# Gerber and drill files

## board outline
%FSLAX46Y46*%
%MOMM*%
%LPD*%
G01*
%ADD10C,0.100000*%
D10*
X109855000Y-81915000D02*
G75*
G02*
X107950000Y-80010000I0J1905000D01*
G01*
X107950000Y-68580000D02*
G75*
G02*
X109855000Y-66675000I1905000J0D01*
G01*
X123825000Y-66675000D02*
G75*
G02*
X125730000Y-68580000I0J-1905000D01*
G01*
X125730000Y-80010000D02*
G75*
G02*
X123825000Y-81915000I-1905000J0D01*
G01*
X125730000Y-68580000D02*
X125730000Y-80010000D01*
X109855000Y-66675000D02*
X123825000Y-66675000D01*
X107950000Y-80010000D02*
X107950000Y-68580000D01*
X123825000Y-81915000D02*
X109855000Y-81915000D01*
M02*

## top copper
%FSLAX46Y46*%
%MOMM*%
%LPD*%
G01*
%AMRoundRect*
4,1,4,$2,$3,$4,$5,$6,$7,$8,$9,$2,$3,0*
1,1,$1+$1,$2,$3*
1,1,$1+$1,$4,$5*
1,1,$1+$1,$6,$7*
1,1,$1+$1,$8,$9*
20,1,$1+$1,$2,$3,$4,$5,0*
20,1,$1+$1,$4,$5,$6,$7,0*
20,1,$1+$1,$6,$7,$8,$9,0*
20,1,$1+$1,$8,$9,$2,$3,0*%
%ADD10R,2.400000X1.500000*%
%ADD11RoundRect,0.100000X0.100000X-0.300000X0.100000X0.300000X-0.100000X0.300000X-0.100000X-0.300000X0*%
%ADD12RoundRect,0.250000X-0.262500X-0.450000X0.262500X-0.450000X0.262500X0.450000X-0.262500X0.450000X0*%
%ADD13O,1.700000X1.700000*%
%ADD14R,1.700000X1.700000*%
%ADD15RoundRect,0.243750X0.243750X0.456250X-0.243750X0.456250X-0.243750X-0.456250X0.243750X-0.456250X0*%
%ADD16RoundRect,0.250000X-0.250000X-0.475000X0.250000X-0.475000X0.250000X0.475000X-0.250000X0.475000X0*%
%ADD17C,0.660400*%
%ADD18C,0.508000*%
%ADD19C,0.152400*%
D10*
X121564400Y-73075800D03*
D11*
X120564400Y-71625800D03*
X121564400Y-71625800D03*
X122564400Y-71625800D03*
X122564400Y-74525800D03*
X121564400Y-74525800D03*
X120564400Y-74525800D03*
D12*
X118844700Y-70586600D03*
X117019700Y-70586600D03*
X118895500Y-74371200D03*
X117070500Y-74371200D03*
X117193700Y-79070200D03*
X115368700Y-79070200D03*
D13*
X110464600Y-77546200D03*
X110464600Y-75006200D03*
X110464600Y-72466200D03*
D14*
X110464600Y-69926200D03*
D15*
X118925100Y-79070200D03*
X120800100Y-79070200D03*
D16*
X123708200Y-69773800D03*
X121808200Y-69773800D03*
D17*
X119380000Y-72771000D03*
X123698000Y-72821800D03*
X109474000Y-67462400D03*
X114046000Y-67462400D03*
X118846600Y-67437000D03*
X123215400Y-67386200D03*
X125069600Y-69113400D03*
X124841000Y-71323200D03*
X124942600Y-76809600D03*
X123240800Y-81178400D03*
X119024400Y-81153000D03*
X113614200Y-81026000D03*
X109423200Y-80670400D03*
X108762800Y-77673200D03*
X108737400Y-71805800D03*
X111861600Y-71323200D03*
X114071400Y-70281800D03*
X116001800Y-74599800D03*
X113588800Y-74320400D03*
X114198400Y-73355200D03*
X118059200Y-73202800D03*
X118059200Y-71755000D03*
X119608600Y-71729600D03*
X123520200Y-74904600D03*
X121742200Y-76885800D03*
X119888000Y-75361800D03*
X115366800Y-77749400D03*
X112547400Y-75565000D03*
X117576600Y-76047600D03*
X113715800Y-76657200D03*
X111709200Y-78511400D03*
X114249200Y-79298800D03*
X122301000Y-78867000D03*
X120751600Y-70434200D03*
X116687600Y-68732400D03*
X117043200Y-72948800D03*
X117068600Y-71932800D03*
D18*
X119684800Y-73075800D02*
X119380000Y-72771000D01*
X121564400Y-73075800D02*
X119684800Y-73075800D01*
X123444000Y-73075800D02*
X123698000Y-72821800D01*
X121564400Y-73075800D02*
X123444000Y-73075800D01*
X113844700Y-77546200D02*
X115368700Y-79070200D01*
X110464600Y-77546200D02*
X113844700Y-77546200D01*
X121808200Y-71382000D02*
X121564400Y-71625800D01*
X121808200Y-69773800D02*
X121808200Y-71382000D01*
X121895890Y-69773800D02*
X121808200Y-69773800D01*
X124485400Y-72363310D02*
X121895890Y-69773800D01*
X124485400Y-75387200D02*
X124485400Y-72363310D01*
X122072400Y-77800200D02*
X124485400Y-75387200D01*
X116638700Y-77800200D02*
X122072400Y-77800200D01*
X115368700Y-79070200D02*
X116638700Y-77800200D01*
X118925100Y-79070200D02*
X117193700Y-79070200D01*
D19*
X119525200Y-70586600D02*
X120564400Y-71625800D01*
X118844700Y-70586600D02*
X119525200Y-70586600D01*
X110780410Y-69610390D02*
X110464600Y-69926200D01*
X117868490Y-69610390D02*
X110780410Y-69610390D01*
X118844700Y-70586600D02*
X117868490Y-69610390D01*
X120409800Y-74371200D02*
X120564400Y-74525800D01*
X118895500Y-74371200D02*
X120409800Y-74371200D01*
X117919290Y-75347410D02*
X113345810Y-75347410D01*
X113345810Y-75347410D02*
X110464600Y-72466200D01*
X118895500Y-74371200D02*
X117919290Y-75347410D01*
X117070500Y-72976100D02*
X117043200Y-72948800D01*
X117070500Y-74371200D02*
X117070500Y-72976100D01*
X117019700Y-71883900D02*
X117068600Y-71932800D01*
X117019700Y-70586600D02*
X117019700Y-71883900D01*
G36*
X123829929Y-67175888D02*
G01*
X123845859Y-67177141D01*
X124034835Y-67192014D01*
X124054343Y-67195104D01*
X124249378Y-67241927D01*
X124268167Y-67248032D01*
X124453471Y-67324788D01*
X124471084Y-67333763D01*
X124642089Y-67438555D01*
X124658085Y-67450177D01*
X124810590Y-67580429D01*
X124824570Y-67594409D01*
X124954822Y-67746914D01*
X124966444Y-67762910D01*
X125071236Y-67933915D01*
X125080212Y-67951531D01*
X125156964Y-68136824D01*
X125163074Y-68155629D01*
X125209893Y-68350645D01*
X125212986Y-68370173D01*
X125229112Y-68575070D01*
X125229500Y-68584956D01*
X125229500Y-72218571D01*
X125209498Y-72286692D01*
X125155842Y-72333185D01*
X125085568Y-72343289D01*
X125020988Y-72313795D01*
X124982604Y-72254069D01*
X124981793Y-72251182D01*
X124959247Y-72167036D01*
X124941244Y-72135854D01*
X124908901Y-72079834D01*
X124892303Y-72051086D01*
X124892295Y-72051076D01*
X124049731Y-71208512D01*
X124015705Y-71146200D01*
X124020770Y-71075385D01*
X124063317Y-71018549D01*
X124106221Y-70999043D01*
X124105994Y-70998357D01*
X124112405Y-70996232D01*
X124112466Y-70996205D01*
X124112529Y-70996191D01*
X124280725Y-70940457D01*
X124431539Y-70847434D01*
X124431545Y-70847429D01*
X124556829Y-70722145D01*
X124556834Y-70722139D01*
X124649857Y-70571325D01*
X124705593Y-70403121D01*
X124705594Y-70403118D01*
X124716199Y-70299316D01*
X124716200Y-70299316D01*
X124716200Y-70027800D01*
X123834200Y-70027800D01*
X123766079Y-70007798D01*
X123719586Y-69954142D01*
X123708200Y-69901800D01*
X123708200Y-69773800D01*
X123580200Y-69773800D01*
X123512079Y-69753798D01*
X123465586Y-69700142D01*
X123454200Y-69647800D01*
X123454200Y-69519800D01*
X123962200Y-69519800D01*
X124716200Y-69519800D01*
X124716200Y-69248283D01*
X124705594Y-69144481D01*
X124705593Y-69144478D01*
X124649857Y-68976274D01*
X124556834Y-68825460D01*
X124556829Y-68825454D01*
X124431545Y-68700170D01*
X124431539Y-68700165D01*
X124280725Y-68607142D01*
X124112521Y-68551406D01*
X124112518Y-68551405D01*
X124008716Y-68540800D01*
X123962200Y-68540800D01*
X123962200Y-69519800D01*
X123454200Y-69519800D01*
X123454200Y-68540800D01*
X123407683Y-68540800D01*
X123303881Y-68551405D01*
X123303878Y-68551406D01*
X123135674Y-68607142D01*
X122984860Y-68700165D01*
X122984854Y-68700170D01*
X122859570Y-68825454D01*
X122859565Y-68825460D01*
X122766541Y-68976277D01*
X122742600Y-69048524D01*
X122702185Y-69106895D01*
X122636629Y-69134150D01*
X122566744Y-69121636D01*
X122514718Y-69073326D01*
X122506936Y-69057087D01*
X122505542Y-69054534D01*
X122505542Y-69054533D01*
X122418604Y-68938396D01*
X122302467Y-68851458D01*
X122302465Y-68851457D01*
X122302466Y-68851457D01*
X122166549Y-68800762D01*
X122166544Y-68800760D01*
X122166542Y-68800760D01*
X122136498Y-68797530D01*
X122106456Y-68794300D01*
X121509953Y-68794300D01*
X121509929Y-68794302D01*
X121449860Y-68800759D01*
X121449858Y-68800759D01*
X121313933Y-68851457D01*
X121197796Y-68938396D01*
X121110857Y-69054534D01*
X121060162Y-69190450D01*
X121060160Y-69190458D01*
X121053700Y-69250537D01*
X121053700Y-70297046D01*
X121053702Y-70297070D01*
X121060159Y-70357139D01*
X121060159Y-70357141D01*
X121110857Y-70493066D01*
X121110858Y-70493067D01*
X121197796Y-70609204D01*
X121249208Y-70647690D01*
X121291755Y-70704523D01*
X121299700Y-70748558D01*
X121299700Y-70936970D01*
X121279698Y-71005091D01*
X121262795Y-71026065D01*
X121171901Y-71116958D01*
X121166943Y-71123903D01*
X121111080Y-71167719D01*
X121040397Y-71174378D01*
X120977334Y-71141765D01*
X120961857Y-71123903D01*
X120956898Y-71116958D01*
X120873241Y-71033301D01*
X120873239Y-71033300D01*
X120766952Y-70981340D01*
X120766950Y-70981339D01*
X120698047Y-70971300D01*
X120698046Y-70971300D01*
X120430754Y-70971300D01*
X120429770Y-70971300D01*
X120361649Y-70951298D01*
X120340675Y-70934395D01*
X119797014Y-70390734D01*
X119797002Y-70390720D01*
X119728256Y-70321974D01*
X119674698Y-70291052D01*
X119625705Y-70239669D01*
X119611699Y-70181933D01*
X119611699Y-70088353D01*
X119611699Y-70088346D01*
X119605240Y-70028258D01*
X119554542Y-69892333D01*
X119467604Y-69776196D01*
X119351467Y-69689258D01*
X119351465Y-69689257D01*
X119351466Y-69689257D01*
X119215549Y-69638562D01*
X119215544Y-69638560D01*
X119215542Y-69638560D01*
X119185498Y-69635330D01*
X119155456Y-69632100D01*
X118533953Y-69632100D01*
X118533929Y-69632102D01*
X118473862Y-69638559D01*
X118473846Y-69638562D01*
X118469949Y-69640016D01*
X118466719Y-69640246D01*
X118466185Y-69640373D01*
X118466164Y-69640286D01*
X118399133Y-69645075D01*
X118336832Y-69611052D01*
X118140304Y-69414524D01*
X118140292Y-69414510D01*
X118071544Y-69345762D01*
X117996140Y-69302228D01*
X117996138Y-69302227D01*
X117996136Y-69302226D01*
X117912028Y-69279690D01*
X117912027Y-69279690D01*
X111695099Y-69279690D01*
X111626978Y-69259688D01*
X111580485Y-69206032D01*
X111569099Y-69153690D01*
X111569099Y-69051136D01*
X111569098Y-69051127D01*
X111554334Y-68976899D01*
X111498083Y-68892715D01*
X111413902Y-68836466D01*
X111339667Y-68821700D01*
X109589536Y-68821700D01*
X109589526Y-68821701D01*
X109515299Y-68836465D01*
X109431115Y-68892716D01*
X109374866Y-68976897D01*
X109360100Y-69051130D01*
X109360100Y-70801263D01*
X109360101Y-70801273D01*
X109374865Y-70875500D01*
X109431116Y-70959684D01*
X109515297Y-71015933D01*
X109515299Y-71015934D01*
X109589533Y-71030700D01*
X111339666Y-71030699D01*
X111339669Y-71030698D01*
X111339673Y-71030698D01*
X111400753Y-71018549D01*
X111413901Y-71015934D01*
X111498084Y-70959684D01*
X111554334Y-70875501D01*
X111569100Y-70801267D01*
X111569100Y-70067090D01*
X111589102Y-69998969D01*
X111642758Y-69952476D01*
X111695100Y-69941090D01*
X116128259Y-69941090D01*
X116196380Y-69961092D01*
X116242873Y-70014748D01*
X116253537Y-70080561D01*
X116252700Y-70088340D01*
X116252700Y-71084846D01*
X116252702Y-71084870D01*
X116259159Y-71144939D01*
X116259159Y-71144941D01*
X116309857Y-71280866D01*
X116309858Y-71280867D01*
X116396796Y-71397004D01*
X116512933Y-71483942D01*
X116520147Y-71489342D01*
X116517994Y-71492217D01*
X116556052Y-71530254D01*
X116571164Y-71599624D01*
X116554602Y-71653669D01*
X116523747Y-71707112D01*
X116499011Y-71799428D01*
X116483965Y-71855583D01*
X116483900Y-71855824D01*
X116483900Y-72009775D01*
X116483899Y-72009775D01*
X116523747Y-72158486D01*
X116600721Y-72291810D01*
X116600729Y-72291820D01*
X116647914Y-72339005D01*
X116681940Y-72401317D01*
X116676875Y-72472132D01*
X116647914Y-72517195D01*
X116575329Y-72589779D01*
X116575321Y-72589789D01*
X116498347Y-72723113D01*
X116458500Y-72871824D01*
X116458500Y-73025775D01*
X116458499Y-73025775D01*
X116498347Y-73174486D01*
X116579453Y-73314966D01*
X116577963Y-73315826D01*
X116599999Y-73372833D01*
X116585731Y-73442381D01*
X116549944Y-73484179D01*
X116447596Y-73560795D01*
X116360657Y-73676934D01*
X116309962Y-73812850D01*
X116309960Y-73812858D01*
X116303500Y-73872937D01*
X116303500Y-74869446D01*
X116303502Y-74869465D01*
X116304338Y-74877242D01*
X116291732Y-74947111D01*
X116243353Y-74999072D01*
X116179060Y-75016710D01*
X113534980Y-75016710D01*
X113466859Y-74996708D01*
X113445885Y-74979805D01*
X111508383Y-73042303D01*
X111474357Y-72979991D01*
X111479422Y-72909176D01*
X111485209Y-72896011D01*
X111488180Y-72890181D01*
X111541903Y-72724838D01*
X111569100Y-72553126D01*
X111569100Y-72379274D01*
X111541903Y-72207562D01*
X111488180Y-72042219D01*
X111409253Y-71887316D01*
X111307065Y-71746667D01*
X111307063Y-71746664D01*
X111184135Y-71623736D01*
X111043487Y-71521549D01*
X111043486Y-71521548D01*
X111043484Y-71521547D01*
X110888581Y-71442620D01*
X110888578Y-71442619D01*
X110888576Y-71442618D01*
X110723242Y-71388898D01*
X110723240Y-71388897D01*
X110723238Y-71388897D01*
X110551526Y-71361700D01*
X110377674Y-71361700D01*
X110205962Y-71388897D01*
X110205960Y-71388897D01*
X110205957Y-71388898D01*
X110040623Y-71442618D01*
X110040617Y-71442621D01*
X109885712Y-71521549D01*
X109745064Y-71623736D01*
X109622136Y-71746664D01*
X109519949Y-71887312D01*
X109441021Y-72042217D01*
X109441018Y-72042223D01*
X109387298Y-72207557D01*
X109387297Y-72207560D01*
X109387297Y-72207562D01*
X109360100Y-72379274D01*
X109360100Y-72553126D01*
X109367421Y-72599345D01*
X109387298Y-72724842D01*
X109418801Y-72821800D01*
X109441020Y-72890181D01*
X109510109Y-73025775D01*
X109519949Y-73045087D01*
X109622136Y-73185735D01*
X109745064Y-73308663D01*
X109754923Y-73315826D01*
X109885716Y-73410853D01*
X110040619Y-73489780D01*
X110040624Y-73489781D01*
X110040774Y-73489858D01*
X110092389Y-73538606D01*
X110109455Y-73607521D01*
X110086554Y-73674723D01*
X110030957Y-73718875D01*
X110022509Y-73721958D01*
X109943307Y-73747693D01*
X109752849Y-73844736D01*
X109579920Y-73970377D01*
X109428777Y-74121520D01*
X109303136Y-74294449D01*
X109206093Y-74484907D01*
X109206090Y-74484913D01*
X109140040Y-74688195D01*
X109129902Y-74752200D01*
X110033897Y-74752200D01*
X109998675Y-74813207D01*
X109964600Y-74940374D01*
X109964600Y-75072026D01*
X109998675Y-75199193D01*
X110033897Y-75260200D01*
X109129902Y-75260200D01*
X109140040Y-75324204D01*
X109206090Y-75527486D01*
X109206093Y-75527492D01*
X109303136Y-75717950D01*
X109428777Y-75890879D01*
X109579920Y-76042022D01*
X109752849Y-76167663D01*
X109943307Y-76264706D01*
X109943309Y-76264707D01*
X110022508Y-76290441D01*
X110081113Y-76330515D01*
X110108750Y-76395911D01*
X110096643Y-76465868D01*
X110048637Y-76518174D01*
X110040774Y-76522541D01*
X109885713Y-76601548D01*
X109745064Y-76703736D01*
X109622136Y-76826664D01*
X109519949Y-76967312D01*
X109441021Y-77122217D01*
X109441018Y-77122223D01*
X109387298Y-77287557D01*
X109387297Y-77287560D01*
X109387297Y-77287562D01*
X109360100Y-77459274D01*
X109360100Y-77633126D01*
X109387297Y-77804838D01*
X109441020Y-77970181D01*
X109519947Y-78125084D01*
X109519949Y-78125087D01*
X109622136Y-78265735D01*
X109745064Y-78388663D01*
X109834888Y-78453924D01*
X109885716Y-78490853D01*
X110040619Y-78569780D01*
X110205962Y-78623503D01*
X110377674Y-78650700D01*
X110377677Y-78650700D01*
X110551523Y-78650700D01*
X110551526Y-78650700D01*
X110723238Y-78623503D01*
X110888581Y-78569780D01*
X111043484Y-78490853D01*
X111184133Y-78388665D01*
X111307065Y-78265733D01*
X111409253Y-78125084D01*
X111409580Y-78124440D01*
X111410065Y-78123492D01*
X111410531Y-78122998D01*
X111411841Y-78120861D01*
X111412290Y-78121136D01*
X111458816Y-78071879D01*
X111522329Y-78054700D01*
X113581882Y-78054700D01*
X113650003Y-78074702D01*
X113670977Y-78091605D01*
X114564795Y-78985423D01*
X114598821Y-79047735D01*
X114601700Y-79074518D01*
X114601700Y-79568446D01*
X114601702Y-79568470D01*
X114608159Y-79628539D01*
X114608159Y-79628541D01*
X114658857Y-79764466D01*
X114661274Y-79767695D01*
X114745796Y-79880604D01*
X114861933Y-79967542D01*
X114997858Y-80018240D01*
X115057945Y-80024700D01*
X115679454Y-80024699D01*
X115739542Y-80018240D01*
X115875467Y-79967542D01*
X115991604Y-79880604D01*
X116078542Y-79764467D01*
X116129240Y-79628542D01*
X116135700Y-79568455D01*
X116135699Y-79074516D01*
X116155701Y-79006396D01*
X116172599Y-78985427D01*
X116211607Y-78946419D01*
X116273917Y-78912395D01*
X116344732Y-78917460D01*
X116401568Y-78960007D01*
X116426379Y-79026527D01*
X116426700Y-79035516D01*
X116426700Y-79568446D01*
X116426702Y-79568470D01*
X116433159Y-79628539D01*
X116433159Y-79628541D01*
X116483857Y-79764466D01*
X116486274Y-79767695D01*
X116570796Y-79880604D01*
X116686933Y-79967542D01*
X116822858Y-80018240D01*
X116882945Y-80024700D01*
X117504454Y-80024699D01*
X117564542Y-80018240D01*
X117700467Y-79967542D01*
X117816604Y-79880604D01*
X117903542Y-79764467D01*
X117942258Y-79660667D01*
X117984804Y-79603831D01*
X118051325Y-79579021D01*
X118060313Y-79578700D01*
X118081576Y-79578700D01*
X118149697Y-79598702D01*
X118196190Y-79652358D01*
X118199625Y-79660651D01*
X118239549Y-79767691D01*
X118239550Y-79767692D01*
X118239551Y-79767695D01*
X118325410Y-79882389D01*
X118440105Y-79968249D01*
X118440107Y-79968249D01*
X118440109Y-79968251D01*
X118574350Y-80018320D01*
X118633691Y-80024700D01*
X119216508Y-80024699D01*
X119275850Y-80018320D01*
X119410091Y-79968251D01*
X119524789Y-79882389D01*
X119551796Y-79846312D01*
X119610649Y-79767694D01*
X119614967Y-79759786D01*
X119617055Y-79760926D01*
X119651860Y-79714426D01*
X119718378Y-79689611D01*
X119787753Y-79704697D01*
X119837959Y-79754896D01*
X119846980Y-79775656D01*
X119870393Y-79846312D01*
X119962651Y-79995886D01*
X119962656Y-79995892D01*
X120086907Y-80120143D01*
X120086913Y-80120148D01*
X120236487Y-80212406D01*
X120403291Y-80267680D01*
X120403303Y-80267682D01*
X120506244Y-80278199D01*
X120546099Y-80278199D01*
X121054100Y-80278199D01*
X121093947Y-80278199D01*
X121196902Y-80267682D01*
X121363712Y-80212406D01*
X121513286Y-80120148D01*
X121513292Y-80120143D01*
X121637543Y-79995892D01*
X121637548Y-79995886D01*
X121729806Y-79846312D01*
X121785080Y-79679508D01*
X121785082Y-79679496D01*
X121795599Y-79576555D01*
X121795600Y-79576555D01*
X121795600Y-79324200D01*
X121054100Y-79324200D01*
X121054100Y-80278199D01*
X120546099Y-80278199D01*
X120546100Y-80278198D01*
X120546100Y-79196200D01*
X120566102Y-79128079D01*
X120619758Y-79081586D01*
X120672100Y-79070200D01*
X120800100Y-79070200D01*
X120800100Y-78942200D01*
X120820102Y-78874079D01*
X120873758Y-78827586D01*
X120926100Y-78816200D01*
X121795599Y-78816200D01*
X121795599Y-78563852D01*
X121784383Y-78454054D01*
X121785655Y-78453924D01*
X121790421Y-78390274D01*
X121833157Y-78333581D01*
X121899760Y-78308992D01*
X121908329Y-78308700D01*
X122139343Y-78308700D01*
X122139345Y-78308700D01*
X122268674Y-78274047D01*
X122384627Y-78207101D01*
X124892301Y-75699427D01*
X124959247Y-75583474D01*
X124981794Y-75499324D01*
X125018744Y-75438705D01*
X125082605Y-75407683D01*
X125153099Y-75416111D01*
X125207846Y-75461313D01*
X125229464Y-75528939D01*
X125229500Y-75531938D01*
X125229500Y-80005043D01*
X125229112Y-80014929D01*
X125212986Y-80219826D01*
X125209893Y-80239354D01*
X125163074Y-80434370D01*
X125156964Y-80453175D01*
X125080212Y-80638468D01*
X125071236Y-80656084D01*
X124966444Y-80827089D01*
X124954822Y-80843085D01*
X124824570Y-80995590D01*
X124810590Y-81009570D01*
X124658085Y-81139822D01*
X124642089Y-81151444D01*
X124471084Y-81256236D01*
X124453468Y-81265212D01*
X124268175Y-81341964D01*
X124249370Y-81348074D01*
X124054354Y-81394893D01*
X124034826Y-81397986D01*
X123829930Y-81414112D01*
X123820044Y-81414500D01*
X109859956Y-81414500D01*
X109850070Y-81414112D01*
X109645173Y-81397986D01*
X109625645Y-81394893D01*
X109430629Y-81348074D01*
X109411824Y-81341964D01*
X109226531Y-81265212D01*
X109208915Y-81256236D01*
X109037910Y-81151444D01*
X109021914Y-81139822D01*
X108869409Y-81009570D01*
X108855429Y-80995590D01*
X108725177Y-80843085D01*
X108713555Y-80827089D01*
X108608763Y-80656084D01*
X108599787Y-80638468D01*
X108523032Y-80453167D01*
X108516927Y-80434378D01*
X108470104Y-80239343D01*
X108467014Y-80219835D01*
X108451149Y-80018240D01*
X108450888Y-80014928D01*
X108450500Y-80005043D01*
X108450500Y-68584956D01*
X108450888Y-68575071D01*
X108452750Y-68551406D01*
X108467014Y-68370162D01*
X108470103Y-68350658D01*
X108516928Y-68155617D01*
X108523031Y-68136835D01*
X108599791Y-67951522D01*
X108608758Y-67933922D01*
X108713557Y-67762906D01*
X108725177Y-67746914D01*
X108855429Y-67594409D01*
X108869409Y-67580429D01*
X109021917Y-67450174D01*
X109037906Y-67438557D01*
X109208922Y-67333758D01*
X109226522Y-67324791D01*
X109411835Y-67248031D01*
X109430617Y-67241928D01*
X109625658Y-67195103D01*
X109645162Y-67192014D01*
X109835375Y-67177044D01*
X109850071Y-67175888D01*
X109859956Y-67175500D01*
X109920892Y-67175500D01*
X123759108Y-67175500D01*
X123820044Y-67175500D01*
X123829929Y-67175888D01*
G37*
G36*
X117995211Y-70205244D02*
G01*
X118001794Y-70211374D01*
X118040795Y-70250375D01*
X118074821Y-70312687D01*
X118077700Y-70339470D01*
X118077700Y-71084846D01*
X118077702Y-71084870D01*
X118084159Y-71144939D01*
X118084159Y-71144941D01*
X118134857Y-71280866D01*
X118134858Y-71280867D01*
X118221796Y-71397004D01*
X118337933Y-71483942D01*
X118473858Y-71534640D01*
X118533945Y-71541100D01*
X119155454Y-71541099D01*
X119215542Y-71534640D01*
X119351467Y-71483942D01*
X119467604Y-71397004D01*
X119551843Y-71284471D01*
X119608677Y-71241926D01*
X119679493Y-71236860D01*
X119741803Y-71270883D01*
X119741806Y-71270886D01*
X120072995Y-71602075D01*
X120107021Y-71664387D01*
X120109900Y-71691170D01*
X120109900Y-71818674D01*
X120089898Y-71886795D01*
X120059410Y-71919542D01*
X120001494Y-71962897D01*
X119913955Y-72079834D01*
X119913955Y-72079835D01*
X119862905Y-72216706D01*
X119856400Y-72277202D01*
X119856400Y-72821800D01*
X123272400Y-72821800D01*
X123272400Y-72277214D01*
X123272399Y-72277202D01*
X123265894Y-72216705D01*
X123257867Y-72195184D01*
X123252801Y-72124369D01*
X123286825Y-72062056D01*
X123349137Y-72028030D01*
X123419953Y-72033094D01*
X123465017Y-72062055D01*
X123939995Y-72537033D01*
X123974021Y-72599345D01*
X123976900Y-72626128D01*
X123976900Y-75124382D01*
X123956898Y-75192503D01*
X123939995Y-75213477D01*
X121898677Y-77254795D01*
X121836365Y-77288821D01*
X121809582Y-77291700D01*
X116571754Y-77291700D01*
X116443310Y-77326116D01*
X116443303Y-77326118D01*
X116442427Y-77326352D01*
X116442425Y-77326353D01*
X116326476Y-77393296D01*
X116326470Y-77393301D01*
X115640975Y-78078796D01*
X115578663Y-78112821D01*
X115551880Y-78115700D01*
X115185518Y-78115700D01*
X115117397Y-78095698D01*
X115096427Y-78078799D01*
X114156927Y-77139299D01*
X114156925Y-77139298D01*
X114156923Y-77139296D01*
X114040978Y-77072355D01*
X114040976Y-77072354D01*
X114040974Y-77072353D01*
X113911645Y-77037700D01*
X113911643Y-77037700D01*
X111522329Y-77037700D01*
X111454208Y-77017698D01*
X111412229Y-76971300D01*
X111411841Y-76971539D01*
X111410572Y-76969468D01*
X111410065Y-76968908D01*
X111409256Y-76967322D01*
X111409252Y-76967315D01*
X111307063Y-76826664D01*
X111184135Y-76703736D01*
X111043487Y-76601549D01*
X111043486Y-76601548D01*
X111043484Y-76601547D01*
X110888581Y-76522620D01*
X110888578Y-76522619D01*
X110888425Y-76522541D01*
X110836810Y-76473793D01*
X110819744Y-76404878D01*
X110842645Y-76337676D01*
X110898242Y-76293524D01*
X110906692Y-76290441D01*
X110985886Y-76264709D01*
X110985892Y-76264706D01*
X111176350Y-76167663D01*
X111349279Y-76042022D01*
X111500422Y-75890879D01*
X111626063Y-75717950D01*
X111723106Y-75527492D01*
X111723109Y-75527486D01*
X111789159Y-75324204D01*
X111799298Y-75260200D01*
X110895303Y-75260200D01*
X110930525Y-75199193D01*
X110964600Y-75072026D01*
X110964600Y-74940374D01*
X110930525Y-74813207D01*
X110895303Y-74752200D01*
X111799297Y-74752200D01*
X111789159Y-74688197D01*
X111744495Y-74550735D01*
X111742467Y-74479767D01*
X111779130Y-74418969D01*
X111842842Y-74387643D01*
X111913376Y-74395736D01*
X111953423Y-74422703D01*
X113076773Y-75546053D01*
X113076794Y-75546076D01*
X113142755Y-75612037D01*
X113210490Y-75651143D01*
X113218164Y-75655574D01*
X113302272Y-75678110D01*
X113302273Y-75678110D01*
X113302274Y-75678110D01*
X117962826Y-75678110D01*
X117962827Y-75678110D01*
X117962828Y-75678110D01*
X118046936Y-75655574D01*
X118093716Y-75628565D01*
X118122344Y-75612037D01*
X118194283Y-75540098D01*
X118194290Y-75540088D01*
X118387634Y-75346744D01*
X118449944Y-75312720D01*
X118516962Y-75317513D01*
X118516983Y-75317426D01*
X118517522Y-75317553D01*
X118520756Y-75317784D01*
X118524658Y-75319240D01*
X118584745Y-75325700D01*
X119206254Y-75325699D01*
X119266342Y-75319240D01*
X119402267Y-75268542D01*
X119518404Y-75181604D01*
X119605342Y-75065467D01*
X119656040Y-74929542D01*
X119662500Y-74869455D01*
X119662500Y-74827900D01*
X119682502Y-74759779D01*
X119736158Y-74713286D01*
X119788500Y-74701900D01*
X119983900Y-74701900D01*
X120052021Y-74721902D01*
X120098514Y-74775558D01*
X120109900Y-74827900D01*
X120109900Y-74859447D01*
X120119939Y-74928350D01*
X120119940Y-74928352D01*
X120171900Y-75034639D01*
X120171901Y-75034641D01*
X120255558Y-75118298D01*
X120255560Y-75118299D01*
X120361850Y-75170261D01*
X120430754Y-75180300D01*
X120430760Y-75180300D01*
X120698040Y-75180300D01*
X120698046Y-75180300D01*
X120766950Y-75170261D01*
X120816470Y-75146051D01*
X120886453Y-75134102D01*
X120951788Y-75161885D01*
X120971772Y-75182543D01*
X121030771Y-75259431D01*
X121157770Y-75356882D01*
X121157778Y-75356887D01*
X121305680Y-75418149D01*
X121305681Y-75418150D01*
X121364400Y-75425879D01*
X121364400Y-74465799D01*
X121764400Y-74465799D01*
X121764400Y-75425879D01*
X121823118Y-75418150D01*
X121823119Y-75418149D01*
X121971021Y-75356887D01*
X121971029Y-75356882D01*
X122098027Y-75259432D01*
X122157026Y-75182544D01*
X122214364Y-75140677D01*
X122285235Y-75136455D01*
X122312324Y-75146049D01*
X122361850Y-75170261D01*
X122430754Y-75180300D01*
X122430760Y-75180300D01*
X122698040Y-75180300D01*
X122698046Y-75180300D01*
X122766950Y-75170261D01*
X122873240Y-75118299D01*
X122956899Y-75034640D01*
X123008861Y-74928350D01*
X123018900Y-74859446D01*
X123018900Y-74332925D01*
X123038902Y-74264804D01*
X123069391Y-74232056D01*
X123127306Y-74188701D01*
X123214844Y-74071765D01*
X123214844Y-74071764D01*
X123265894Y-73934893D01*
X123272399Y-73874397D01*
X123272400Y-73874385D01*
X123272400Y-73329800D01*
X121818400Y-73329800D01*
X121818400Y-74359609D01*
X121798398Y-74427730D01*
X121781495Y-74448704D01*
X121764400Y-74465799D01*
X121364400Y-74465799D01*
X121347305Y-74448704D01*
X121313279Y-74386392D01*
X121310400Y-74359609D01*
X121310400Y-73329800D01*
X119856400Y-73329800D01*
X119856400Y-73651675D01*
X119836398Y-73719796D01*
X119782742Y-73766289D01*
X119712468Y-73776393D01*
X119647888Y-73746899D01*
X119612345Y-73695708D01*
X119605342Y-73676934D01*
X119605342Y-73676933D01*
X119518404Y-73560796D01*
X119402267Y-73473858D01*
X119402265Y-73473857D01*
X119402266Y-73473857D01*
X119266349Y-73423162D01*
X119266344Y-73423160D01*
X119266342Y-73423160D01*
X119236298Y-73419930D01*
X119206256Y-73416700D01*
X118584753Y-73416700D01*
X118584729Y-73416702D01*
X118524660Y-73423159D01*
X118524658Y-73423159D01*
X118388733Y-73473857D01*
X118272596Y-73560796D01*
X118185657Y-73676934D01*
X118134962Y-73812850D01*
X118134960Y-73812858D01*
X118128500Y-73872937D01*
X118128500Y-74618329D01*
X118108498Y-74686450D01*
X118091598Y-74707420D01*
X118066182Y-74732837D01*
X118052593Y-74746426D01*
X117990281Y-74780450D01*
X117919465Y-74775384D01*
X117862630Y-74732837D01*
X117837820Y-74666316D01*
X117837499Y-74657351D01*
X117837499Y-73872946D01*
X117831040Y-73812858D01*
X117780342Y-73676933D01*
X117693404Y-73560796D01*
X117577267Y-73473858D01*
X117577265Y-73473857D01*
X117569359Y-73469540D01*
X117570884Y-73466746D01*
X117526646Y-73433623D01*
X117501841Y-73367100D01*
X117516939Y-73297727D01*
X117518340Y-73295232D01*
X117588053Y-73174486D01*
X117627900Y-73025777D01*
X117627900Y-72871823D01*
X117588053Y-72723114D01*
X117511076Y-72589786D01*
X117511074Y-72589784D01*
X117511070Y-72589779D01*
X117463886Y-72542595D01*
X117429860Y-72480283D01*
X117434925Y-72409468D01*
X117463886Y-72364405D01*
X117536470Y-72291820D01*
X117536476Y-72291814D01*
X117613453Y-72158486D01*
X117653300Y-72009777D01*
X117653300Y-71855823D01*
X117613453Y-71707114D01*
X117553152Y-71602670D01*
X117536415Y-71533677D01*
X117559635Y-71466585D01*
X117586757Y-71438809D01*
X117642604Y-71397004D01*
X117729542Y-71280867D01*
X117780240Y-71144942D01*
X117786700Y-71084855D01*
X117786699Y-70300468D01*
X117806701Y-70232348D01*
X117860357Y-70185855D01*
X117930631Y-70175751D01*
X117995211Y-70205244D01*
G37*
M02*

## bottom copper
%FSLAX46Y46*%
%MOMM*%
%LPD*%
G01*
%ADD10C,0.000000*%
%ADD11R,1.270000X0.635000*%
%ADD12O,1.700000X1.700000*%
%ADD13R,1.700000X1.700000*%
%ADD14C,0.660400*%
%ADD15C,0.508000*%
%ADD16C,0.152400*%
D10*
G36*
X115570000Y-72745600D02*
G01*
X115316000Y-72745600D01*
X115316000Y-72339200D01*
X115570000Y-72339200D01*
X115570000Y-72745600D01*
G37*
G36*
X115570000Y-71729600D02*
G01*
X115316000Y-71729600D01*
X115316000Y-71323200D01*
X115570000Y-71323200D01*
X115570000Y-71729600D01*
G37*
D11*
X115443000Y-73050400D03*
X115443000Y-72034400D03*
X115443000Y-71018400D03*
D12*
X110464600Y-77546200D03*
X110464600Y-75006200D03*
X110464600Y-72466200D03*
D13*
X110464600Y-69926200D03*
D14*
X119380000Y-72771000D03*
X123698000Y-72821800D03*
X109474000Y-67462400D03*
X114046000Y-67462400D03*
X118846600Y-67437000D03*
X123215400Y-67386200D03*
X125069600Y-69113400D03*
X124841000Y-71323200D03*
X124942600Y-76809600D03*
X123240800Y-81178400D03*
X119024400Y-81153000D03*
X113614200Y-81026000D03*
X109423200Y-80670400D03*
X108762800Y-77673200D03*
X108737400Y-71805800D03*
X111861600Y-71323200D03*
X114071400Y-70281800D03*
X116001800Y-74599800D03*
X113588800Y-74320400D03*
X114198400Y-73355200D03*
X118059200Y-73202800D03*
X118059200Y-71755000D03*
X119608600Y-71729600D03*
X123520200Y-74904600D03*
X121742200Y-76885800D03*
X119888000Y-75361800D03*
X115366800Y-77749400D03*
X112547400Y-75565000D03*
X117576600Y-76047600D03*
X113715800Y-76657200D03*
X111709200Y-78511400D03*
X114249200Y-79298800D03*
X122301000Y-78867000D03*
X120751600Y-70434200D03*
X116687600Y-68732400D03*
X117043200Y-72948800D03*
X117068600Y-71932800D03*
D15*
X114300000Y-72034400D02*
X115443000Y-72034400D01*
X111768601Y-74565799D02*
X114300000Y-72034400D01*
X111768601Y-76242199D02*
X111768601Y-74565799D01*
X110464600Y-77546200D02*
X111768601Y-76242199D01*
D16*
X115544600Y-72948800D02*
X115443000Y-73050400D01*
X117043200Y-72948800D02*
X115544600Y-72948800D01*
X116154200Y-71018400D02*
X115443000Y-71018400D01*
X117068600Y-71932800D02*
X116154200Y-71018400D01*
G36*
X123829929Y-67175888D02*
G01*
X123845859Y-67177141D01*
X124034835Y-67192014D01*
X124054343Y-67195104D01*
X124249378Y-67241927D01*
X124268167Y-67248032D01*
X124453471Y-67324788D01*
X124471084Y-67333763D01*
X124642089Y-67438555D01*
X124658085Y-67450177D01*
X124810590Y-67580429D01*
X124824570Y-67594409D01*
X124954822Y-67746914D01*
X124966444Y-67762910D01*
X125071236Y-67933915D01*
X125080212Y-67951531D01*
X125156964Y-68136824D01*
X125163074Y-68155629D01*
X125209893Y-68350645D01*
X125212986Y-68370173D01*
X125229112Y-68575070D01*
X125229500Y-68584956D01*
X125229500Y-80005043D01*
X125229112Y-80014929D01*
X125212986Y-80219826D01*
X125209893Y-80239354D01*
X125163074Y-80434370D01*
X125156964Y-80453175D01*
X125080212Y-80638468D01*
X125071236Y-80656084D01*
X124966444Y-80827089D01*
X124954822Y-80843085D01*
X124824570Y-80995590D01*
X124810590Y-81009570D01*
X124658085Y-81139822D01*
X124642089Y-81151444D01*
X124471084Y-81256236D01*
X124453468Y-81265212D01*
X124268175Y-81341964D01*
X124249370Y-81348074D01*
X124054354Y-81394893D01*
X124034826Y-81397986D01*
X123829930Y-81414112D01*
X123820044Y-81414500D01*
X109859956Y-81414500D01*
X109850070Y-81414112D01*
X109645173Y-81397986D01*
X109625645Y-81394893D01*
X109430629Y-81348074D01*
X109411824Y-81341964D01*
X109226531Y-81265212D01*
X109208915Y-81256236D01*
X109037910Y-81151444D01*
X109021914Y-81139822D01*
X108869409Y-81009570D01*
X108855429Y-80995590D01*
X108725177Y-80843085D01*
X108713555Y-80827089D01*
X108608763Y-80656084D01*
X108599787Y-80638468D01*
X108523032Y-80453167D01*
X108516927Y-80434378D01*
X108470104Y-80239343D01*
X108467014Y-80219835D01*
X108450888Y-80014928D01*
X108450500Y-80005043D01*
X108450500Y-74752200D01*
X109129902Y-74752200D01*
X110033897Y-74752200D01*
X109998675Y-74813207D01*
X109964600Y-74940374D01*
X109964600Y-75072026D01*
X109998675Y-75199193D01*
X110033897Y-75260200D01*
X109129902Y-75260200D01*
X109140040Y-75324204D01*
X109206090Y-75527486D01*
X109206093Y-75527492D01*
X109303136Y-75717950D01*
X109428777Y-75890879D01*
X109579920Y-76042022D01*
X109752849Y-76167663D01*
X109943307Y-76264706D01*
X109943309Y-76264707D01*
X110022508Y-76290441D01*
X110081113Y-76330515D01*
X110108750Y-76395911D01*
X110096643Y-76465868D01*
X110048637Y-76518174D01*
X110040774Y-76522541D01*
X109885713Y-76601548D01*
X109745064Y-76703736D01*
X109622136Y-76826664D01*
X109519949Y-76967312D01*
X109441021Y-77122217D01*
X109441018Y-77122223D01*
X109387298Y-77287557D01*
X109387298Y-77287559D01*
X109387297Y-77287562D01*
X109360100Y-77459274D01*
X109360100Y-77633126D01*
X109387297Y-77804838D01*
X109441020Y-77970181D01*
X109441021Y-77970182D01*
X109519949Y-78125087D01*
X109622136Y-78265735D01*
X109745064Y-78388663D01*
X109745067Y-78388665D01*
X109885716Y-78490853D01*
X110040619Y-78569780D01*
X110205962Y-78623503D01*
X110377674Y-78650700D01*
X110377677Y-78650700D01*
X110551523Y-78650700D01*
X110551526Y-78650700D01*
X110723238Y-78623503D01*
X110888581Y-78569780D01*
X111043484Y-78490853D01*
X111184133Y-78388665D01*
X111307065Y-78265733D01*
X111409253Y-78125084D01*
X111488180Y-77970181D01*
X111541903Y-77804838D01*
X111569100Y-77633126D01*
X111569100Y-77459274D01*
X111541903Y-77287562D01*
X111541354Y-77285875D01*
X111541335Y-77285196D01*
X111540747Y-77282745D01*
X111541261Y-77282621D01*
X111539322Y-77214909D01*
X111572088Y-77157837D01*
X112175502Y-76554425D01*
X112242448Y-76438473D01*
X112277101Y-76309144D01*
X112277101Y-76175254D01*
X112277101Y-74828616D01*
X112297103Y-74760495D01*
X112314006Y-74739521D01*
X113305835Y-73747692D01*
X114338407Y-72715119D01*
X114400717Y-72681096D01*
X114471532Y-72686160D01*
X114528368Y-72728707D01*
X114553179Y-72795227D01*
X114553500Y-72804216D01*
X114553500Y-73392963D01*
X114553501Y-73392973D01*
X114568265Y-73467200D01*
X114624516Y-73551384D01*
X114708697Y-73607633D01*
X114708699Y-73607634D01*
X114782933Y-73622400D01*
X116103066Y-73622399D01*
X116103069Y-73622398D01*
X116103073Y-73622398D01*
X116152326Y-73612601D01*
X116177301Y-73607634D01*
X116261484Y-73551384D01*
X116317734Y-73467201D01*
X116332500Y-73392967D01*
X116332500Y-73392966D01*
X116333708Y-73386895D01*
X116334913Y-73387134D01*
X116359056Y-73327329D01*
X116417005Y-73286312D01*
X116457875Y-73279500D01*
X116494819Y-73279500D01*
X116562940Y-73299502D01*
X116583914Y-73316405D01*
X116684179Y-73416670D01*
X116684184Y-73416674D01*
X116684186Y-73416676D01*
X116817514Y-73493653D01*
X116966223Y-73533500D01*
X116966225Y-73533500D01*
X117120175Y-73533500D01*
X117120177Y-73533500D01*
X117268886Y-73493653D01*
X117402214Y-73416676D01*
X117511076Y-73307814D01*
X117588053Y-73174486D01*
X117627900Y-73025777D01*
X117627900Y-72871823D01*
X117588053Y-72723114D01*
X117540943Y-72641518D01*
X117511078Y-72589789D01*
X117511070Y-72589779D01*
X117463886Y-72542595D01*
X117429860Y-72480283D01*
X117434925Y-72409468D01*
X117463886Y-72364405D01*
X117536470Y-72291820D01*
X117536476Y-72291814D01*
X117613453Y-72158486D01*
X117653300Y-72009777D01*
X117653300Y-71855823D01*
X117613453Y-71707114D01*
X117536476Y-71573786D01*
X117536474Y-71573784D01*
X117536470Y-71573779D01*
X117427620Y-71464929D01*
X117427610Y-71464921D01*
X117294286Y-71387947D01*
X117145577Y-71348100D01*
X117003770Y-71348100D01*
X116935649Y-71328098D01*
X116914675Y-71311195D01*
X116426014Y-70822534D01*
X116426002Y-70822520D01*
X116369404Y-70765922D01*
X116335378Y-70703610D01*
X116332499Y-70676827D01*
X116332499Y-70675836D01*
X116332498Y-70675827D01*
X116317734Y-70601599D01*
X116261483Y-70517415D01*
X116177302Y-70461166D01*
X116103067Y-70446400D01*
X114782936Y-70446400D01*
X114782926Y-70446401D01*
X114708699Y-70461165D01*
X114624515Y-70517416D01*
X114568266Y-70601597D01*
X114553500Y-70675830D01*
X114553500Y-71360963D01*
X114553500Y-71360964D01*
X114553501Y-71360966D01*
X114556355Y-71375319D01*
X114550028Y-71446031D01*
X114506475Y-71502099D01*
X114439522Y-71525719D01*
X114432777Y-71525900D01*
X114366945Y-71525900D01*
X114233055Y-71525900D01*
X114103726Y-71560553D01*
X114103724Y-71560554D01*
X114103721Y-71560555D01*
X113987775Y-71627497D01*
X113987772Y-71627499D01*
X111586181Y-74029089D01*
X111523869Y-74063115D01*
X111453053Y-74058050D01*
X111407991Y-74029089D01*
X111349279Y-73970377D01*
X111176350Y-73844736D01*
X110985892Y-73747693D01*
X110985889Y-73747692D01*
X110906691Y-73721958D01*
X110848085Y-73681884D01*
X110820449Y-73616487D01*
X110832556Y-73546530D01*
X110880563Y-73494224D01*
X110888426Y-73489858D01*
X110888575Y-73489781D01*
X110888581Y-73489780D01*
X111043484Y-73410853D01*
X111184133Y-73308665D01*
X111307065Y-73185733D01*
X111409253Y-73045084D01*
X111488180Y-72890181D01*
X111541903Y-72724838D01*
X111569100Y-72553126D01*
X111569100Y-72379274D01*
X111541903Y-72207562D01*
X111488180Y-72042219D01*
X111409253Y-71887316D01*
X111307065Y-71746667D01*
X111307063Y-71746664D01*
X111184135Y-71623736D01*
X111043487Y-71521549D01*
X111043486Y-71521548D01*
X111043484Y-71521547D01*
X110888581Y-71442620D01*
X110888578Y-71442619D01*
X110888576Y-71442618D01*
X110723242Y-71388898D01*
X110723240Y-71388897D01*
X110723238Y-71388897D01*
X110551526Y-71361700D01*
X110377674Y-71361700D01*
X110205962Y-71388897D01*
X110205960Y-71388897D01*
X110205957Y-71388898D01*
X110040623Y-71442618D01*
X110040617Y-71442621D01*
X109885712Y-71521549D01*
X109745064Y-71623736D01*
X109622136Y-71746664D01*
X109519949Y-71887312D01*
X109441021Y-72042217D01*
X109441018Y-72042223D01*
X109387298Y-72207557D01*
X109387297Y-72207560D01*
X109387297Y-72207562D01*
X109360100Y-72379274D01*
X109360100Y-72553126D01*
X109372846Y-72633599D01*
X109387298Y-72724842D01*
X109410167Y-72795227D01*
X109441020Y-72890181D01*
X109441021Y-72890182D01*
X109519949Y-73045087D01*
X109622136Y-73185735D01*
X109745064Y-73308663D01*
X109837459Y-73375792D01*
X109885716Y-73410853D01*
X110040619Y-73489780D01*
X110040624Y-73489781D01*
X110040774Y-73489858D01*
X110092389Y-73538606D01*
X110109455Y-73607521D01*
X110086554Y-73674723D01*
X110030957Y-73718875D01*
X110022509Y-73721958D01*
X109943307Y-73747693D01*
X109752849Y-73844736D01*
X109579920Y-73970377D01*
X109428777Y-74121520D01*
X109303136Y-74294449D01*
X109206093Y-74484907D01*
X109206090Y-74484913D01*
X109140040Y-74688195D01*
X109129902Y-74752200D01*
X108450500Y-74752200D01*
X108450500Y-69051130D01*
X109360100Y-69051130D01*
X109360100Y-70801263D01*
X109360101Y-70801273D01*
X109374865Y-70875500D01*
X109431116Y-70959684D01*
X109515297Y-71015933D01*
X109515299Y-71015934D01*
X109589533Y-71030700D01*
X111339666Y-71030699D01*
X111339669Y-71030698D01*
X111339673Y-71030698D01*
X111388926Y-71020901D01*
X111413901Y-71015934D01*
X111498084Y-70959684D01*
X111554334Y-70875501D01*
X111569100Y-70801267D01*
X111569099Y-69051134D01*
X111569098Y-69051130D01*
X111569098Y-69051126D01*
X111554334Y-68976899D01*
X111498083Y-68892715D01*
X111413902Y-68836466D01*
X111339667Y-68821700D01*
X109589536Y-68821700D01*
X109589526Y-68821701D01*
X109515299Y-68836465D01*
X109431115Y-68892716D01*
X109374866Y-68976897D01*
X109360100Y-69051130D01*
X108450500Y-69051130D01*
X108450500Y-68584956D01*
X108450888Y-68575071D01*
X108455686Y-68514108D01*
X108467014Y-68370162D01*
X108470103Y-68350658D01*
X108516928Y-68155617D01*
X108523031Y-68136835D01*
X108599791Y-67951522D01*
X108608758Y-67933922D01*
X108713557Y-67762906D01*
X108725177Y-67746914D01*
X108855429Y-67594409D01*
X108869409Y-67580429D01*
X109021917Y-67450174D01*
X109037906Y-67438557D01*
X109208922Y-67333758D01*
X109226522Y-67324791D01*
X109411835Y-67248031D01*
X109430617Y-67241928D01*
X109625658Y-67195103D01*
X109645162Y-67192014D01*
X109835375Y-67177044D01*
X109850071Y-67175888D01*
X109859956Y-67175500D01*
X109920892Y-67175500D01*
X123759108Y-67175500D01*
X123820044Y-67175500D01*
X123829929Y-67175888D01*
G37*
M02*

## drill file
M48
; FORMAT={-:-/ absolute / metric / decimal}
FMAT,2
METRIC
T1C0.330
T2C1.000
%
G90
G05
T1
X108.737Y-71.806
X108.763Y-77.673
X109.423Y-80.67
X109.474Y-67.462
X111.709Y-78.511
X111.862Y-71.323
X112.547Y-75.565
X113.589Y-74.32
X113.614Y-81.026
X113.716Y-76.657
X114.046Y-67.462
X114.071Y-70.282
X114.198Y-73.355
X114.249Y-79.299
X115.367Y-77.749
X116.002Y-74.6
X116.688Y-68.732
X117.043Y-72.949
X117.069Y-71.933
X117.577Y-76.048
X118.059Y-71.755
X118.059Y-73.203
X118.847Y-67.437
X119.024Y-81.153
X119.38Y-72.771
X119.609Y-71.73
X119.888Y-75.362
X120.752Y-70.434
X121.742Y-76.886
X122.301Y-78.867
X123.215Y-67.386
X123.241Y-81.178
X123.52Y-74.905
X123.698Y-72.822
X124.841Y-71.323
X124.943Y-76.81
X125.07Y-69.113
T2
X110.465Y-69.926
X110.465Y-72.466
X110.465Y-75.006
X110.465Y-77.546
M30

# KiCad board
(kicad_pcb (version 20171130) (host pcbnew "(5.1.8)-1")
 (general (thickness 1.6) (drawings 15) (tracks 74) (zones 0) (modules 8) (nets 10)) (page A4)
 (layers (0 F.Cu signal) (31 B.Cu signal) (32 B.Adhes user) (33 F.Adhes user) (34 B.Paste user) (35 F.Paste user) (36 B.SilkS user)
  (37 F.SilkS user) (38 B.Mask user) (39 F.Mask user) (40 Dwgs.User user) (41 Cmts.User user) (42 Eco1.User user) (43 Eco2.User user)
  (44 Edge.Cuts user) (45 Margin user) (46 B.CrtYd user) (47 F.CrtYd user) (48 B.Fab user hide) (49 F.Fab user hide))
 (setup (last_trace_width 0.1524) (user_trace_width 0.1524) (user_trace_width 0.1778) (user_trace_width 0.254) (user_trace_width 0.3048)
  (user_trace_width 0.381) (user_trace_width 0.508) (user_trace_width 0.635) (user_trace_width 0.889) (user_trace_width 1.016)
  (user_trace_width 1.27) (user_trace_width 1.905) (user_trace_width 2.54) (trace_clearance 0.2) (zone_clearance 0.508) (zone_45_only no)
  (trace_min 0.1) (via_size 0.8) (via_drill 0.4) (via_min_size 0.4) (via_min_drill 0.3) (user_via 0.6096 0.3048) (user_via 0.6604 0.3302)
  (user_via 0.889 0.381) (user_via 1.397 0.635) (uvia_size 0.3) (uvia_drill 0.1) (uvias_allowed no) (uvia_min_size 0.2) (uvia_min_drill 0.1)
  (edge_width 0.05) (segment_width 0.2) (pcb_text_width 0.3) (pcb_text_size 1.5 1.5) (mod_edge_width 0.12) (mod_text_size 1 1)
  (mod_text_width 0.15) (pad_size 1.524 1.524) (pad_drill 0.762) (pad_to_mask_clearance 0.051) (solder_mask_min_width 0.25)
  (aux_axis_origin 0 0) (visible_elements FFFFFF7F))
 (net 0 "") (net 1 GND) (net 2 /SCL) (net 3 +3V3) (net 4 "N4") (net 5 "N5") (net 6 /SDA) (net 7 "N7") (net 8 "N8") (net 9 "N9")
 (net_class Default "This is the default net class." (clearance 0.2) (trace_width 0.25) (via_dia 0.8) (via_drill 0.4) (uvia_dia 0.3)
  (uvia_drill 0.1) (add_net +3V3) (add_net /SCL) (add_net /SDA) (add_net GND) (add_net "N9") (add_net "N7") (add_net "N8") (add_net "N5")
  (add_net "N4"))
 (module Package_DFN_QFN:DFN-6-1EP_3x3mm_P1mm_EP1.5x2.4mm (layer F.Cu) (at 121.5644 73.0758 90)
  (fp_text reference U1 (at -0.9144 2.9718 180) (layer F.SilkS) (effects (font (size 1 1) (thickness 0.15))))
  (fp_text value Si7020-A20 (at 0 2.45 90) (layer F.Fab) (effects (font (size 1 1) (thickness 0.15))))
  (pad "" smd roundrect (at 0.375 0.6 90) (size 0.6 0.97) (layers F.Paste) (roundrect_rratio 0.25))
  (pad "" smd roundrect (at 0.375 -0.6 90) (size 0.6 0.97) (layers F.Paste) (roundrect_rratio 0.25))
  (pad "" smd roundrect (at -0.375 0.6 90) (size 0.6 0.97) (layers F.Paste) (roundrect_rratio 0.25))
  (pad "" smd roundrect (at -0.375 -0.6 90) (size 0.6 0.97) (layers F.Paste) (roundrect_rratio 0.25))
  (pad 7 smd rect (at 0 0 90) (size 1.5 2.4) (layers F.Cu F.Mask) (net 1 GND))
  (pad 6 smd roundrect (at 1.45 -1 90) (size 0.8 0.4) (layers F.Cu F.Paste F.Mask) (roundrect_rratio 0.25) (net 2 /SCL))
  (pad 5 smd roundrect (at 1.45 0 90) (size 0.8 0.4) (layers F.Cu F.Paste F.Mask) (roundrect_rratio 0.25) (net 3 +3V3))
  (pad 4 smd roundrect (at 1.45 1 90) (size 0.8 0.4) (layers F.Cu F.Paste F.Mask) (roundrect_rratio 0.25) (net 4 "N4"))
  (pad 3 smd roundrect (at -1.45 1 90) (size 0.8 0.4) (layers F.Cu F.Paste F.Mask) (roundrect_rratio 0.25) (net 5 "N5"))
  (pad 2 smd roundrect (at -1.45 0 90) (size 0.8 0.4) (layers F.Cu F.Paste F.Mask) (roundrect_rratio 0.25) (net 1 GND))
  (pad 1 smd roundrect (at -1.45 -1 90) (size 0.8 0.4) (layers F.Cu F.Paste F.Mask) (roundrect_rratio 0.25) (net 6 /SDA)))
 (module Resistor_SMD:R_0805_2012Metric (layer F.Cu) (at 117.9322 70.5866)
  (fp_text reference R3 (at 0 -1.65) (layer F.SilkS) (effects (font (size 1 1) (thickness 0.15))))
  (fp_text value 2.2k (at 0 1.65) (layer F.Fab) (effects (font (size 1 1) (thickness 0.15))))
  (pad 2 smd roundrect (at 0.9125 0) (size 1.025 1.4) (layers F.Cu F.Paste F.Mask) (roundrect_rratio 0.243902) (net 2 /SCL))
  (pad 1 smd roundrect (at -0.9125 0) (size 1.025 1.4) (layers F.Cu F.Paste F.Mask) (roundrect_rratio 0.243902) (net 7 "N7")))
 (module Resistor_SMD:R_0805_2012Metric (layer F.Cu) (at 117.983 74.3712)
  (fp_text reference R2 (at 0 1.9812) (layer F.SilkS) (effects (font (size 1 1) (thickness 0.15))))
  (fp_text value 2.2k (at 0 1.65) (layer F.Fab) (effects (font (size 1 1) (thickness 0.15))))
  (pad 2 smd roundrect (at 0.9125 0) (size 1.025 1.4) (layers F.Cu F.Paste F.Mask) (roundrect_rratio 0.243902) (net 6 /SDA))
  (pad 1 smd roundrect (at -0.9125 0) (size 1.025 1.4) (layers F.Cu F.Paste F.Mask) (roundrect_rratio 0.243902) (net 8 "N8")))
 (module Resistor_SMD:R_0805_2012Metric (layer F.Cu) (at 116.2812 79.0702)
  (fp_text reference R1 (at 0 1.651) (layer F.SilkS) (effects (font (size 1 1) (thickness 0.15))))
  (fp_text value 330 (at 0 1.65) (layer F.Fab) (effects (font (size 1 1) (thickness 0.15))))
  (pad 2 smd roundrect (at 0.9125 0) (size 1.025 1.4) (layers F.Cu F.Paste F.Mask) (roundrect_rratio 0.243902) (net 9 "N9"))
  (pad 1 smd roundrect (at -0.9125 0) (size 1.025 1.4) (layers F.Cu F.Paste F.Mask) (roundrect_rratio 0.243902) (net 3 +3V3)))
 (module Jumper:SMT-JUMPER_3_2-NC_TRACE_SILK (layer B.Cu) (at 115.443 72.0344 270)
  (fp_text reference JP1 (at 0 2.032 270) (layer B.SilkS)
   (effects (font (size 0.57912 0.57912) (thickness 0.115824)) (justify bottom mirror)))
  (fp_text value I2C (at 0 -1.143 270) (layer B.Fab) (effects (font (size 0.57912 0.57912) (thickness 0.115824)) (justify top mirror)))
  (fp_poly (pts (xy 0.3048 -0.127) (xy 0.7112 -0.127) (xy 0.7112 0.127) (xy 0.3048 0.127)) (layer B.Cu) (width 0))
  (fp_poly (pts (xy -0.7112 -0.127) (xy -0.3048 -0.127) (xy -0.3048 0.127) (xy -0.7112 0.127)) (layer B.Cu) (width 0))
  (pad 3 smd rect (at 1.016 0 270) (size 0.635 1.27) (layers B.Cu B.Mask) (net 8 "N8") (solder_mask_margin 0.1016))
  (pad 2 smd rect (at 0 0 270) (size 0.635 1.27) (layers B.Cu B.Mask) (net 3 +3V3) (solder_mask_margin 0.1016))
  (pad 1 smd rect (at -1.016 0 270) (size 0.635 1.27) (layers B.Cu B.Mask) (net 7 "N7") (solder_mask_margin 0.1016)))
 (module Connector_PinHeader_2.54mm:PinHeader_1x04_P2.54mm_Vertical (layer F.Cu) (at 110.4646 69.9262)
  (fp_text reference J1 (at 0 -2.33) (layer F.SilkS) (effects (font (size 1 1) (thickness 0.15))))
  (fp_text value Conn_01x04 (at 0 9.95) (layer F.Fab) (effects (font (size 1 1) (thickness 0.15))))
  (pad 4 thru_hole oval (at 0 7.62) (size 1.7 1.7) (drill 1) (layers *.Cu *.Mask) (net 3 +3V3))
  (pad 3 thru_hole oval (at 0 5.08) (size 1.7 1.7) (drill 1) (layers *.Cu *.Mask) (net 1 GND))
  (pad 2 thru_hole oval (at 0 2.54) (size 1.7 1.7) (drill 1) (layers *.Cu *.Mask) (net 6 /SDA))
  (pad 1 thru_hole rect (at 0 0) (size 1.7 1.7) (drill 1) (layers *.Cu *.Mask) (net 2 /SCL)))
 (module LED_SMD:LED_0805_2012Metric (layer F.Cu) (at 119.8626 79.0702 180)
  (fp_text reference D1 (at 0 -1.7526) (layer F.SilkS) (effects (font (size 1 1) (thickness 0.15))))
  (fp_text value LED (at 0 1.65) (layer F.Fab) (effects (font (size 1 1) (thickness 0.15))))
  (pad 2 smd roundrect (at 0.9375 0 180) (size 0.975 1.4) (layers F.Cu F.Paste F.Mask) (roundrect_rratio 0.25) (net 9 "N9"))
  (pad 1 smd roundrect (at -0.9375 0 180) (size 0.975 1.4) (layers F.Cu F.Paste F.Mask) (roundrect_rratio 0.25) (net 1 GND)))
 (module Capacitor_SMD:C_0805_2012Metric (layer F.Cu) (at 122.7582 69.7738)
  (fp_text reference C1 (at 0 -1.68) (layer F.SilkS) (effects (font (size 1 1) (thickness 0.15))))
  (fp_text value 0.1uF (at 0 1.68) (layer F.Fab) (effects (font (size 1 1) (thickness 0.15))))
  (pad 2 smd roundrect (at 0.95 0) (size 1 1.45) (layers F.Cu F.Paste F.Mask) (roundrect_rratio 0.25) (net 1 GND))
  (pad 1 smd roundrect (at -0.95 0) (size 1 1.45) (layers F.Cu F.Paste F.Mask) (roundrect_rratio 0.25) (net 3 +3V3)))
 (gr_arc (start 109.855 80.01) (end 107.95 80.01) (angle -90) (layer Edge.Cuts) (width 0.1))
 (gr_arc (start 109.855 68.58) (end 109.855 66.675) (angle -90) (layer Edge.Cuts) (width 0.1))
 (gr_arc (start 123.825 68.58) (end 125.73 68.58) (angle -90) (layer Edge.Cuts) (width 0.1))
 (gr_arc (start 123.825 80.01) (end 123.825 81.915) (angle -90) (layer Edge.Cuts) (width 0.1))
 (gr_line (start 125.73 68.58) (end 125.73 80.01) (layer Edge.Cuts) (width 0.1))
 (gr_line (start 109.855 66.675) (end 123.825 66.675) (layer Edge.Cuts) (width 0.1))
 (gr_line (start 107.95 80.01) (end 107.95 68.58) (layer Edge.Cuts) (width 0.1))
 (gr_line (start 123.825 81.915) (end 109.855 81.915) (layer Edge.Cuts) (width 0.1))
 (via (at 119.38 72.771) (size 0.6604) (drill 0.3302) (layers F.Cu B.Cu) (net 1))
 (via (at 123.698 72.8218) (size 0.6604) (drill 0.3302) (layers F.Cu B.Cu) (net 1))
 (segment (start 119.6848 73.0758) (end 119.38 72.771) (width 0.508) (layer F.Cu) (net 1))
 (segment (start 121.5644 73.0758) (end 119.6848 73.0758) (width 0.508) (layer F.Cu) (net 1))
 (segment (start 123.444 73.0758) (end 123.698 72.8218) (width 0.508) (layer F.Cu) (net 1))
 (segment (start 121.5644 73.0758) (end 123.444 73.0758) (width 0.508) (layer F.Cu) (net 1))
 (via (at 109.474 67.4624) (size 0.6604) (drill 0.3302) (layers F.Cu B.Cu) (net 1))
 (via (at 114.046 67.4624) (size 0.6604) (drill 0.3302) (layers F.Cu B.Cu) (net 1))
 (via (at 118.8466 67.437) (size 0.6604) (drill 0.3302) (layers F.Cu B.Cu) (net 1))
 (via (at 123.2154 67.3862) (size 0.6604) (drill 0.3302) (layers F.Cu B.Cu) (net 1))
 (via (at 125.0696 69.1134) (size 0.6604) (drill 0.3302) (layers F.Cu B.Cu) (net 1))
 (via (at 124.841 71.3232) (size 0.6604) (drill 0.3302) (layers F.Cu B.Cu) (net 1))
 (via (at 124.9426 76.8096) (size 0.6604) (drill 0.3302) (layers F.Cu B.Cu) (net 1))
 (via (at 123.2408 81.1784) (size 0.6604) (drill 0.3302) (layers F.Cu B.Cu) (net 1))
 (via (at 119.0244 81.153) (size 0.6604) (drill 0.3302) (layers F.Cu B.Cu) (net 1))
 (via (at 113.6142 81.026) (size 0.6604) (drill 0.3302) (layers F.Cu B.Cu) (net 1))
 (via (at 109.4232 80.6704) (size 0.6604) (drill 0.3302) (layers F.Cu B.Cu) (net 1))
 (via (at 108.7628 77.6732) (size 0.6604) (drill 0.3302) (layers F.Cu B.Cu) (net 1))
 (via (at 108.7374 71.8058) (size 0.6604) (drill 0.3302) (layers F.Cu B.Cu) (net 1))
 (via (at 111.8616 71.3232) (size 0.6604) (drill 0.3302) (layers F.Cu B.Cu) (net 1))
 (via (at 114.0714 70.2818) (size 0.6604) (drill 0.3302) (layers F.Cu B.Cu) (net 1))
 (via (at 116.0018 74.5998) (size 0.6604) (drill 0.3302) (layers F.Cu B.Cu) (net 1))
 (via (at 113.5888 74.3204) (size 0.6604) (drill 0.3302) (layers F.Cu B.Cu) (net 1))
 (via (at 114.1984 73.3552) (size 0.6604) (drill 0.3302) (layers F.Cu B.Cu) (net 1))
 (via (at 118.0592 73.2028) (size 0.6604) (drill 0.3302) (layers F.Cu B.Cu) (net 1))
 (via (at 118.0592 71.755) (size 0.6604) (drill 0.3302) (layers F.Cu B.Cu) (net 1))
 (via (at 119.6086 71.7296) (size 0.6604) (drill 0.3302) (layers F.Cu B.Cu) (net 1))
 (via (at 123.5202 74.9046) (size 0.6604) (drill 0.3302) (layers F.Cu B.Cu) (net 1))
 (via (at 121.7422 76.8858) (size 0.6604) (drill 0.3302) (layers F.Cu B.Cu) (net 1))
 (via (at 119.888 75.3618) (size 0.6604) (drill 0.3302) (layers F.Cu B.Cu) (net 1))
 (via (at 115.3668 77.7494) (size 0.6604) (drill 0.3302) (layers F.Cu B.Cu) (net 1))
 (via (at 112.5474 75.565) (size 0.6604) (drill 0.3302) (layers F.Cu B.Cu) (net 1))
 (via (at 117.5766 76.0476) (size 0.6604) (drill 0.3302) (layers F.Cu B.Cu) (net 1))
 (via (at 113.7158 76.6572) (size 0.6604) (drill 0.3302) (layers F.Cu B.Cu) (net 1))
 (via (at 111.7092 78.5114) (size 0.6604) (drill 0.3302) (layers F.Cu B.Cu) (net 1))
 (via (at 114.2492 79.2988) (size 0.6604) (drill 0.3302) (layers F.Cu B.Cu) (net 1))
 (via (at 122.301 78.867) (size 0.6604) (drill 0.3302) (layers F.Cu B.Cu) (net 1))
 (via (at 120.7516 70.4342) (size 0.6604) (drill 0.3302) (layers F.Cu B.Cu) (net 1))
 (via (at 116.6876 68.7324) (size 0.6604) (drill 0.3302) (layers F.Cu B.Cu) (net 1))
 (segment (start 113.8447 77.5462) (end 115.3687 79.0702) (width 0.508) (layer F.Cu) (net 3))
 (segment (start 110.4646 77.5462) (end 113.8447 77.5462) (width 0.508) (layer F.Cu) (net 3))
 (segment (start 121.8082 71.382) (end 121.5644 71.6258) (width 0.508) (layer F.Cu) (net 3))
 (segment (start 121.8082 69.7738) (end 121.8082 71.382) (width 0.508) (layer F.Cu) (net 3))
 (segment (start 114.3 72.0344) (end 115.443 72.0344) (width 0.508) (layer B.Cu) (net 3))
 (segment (start 111.768601 74.565799) (end 114.3 72.0344) (width 0.508) (layer B.Cu) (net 3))
 (segment (start 111.768601 76.242199) (end 111.768601 74.565799) (width 0.508) (layer B.Cu) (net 3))
 (segment (start 110.4646 77.5462) (end 111.768601 76.242199) (width 0.508) (layer B.Cu) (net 3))
 (segment (start 121.89589 69.7738) (end 121.8082 69.7738) (width 0.508) (layer F.Cu) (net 3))
 (segment (start 124.4854 72.36331) (end 121.89589 69.7738) (width 0.508) (layer F.Cu) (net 3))
 (segment (start 124.4854 75.3872) (end 124.4854 72.36331) (width 0.508) (layer F.Cu) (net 3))
 (segment (start 122.0724 77.8002) (end 124.4854 75.3872) (width 0.508) (layer F.Cu) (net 3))
 (segment (start 116.6387 77.8002) (end 122.0724 77.8002) (width 0.508) (layer F.Cu) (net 3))
 (segment (start 115.3687 79.0702) (end 116.6387 77.8002) (width 0.508) (layer F.Cu) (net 3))
 (segment (start 118.9251 79.0702) (end 117.1937 79.0702) (width 0.508) (layer F.Cu) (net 9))
 (segment (start 119.5252 70.5866) (end 120.5644 71.6258) (width 0.1524) (layer F.Cu) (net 2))
 (segment (start 118.8447 70.5866) (end 119.5252 70.5866) (width 0.1524) (layer F.Cu) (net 2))
 (segment (start 110.78041 69.61039) (end 110.4646 69.9262) (width 0.1524) (layer F.Cu) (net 2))
 (segment (start 117.86849 69.61039) (end 110.78041 69.61039) (width 0.1524) (layer F.Cu) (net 2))
 (segment (start 118.8447 70.5866) (end 117.86849 69.61039) (width 0.1524) (layer F.Cu) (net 2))
 (segment (start 120.4098 74.3712) (end 120.5644 74.5258) (width 0.1524) (layer F.Cu) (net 6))
 (segment (start 118.8955 74.3712) (end 120.4098 74.3712) (width 0.1524) (layer F.Cu) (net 6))
 (segment (start 117.91929 75.34741) (end 113.34581 75.34741) (width 0.1524) (layer F.Cu) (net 6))
 (segment (start 113.34581 75.34741) (end 110.4646 72.4662) (width 0.1524) (layer F.Cu) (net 6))
 (segment (start 118.8955 74.3712) (end 117.91929 75.34741) (width 0.1524) (layer F.Cu) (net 6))
 (via (at 117.0432 72.9488) (size 0.6604) (drill 0.3302) (layers F.Cu B.Cu) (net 8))
 (segment (start 117.0705 72.9761) (end 117.0432 72.9488) (width 0.1524) (layer F.Cu) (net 8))
 (segment (start 117.0705 74.3712) (end 117.0705 72.9761) (width 0.1524) (layer F.Cu) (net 8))
 (segment (start 115.5446 72.9488) (end 115.443 73.0504) (width 0.1524) (layer B.Cu) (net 8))
 (segment (start 117.0432 72.9488) (end 115.5446 72.9488) (width 0.1524) (layer B.Cu) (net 8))
 (via (at 117.0686 71.9328) (size 0.6604) (drill 0.3302) (layers F.Cu B.Cu) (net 7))
 (segment (start 117.0197 71.8839) (end 117.0686 71.9328) (width 0.1524) (layer F.Cu) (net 7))
 (segment (start 117.0197 70.5866) (end 117.0197 71.8839) (width 0.1524) (layer F.Cu) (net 7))
 (segment (start 116.1542 71.0184) (end 115.443 71.0184) (width 0.1524) (layer B.Cu) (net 7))
 (segment (start 117.0686 71.9328) (end 116.1542 71.0184) (width 0.1524) (layer B.Cu) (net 7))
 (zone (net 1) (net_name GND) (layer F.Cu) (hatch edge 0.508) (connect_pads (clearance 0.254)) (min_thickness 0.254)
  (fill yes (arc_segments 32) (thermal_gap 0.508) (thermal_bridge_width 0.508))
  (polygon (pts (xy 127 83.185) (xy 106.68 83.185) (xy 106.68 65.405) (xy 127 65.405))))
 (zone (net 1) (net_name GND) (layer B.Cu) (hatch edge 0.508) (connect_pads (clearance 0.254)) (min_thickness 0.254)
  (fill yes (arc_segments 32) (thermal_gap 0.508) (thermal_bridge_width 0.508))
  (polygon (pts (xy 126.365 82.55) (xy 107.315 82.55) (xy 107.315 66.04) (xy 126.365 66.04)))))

